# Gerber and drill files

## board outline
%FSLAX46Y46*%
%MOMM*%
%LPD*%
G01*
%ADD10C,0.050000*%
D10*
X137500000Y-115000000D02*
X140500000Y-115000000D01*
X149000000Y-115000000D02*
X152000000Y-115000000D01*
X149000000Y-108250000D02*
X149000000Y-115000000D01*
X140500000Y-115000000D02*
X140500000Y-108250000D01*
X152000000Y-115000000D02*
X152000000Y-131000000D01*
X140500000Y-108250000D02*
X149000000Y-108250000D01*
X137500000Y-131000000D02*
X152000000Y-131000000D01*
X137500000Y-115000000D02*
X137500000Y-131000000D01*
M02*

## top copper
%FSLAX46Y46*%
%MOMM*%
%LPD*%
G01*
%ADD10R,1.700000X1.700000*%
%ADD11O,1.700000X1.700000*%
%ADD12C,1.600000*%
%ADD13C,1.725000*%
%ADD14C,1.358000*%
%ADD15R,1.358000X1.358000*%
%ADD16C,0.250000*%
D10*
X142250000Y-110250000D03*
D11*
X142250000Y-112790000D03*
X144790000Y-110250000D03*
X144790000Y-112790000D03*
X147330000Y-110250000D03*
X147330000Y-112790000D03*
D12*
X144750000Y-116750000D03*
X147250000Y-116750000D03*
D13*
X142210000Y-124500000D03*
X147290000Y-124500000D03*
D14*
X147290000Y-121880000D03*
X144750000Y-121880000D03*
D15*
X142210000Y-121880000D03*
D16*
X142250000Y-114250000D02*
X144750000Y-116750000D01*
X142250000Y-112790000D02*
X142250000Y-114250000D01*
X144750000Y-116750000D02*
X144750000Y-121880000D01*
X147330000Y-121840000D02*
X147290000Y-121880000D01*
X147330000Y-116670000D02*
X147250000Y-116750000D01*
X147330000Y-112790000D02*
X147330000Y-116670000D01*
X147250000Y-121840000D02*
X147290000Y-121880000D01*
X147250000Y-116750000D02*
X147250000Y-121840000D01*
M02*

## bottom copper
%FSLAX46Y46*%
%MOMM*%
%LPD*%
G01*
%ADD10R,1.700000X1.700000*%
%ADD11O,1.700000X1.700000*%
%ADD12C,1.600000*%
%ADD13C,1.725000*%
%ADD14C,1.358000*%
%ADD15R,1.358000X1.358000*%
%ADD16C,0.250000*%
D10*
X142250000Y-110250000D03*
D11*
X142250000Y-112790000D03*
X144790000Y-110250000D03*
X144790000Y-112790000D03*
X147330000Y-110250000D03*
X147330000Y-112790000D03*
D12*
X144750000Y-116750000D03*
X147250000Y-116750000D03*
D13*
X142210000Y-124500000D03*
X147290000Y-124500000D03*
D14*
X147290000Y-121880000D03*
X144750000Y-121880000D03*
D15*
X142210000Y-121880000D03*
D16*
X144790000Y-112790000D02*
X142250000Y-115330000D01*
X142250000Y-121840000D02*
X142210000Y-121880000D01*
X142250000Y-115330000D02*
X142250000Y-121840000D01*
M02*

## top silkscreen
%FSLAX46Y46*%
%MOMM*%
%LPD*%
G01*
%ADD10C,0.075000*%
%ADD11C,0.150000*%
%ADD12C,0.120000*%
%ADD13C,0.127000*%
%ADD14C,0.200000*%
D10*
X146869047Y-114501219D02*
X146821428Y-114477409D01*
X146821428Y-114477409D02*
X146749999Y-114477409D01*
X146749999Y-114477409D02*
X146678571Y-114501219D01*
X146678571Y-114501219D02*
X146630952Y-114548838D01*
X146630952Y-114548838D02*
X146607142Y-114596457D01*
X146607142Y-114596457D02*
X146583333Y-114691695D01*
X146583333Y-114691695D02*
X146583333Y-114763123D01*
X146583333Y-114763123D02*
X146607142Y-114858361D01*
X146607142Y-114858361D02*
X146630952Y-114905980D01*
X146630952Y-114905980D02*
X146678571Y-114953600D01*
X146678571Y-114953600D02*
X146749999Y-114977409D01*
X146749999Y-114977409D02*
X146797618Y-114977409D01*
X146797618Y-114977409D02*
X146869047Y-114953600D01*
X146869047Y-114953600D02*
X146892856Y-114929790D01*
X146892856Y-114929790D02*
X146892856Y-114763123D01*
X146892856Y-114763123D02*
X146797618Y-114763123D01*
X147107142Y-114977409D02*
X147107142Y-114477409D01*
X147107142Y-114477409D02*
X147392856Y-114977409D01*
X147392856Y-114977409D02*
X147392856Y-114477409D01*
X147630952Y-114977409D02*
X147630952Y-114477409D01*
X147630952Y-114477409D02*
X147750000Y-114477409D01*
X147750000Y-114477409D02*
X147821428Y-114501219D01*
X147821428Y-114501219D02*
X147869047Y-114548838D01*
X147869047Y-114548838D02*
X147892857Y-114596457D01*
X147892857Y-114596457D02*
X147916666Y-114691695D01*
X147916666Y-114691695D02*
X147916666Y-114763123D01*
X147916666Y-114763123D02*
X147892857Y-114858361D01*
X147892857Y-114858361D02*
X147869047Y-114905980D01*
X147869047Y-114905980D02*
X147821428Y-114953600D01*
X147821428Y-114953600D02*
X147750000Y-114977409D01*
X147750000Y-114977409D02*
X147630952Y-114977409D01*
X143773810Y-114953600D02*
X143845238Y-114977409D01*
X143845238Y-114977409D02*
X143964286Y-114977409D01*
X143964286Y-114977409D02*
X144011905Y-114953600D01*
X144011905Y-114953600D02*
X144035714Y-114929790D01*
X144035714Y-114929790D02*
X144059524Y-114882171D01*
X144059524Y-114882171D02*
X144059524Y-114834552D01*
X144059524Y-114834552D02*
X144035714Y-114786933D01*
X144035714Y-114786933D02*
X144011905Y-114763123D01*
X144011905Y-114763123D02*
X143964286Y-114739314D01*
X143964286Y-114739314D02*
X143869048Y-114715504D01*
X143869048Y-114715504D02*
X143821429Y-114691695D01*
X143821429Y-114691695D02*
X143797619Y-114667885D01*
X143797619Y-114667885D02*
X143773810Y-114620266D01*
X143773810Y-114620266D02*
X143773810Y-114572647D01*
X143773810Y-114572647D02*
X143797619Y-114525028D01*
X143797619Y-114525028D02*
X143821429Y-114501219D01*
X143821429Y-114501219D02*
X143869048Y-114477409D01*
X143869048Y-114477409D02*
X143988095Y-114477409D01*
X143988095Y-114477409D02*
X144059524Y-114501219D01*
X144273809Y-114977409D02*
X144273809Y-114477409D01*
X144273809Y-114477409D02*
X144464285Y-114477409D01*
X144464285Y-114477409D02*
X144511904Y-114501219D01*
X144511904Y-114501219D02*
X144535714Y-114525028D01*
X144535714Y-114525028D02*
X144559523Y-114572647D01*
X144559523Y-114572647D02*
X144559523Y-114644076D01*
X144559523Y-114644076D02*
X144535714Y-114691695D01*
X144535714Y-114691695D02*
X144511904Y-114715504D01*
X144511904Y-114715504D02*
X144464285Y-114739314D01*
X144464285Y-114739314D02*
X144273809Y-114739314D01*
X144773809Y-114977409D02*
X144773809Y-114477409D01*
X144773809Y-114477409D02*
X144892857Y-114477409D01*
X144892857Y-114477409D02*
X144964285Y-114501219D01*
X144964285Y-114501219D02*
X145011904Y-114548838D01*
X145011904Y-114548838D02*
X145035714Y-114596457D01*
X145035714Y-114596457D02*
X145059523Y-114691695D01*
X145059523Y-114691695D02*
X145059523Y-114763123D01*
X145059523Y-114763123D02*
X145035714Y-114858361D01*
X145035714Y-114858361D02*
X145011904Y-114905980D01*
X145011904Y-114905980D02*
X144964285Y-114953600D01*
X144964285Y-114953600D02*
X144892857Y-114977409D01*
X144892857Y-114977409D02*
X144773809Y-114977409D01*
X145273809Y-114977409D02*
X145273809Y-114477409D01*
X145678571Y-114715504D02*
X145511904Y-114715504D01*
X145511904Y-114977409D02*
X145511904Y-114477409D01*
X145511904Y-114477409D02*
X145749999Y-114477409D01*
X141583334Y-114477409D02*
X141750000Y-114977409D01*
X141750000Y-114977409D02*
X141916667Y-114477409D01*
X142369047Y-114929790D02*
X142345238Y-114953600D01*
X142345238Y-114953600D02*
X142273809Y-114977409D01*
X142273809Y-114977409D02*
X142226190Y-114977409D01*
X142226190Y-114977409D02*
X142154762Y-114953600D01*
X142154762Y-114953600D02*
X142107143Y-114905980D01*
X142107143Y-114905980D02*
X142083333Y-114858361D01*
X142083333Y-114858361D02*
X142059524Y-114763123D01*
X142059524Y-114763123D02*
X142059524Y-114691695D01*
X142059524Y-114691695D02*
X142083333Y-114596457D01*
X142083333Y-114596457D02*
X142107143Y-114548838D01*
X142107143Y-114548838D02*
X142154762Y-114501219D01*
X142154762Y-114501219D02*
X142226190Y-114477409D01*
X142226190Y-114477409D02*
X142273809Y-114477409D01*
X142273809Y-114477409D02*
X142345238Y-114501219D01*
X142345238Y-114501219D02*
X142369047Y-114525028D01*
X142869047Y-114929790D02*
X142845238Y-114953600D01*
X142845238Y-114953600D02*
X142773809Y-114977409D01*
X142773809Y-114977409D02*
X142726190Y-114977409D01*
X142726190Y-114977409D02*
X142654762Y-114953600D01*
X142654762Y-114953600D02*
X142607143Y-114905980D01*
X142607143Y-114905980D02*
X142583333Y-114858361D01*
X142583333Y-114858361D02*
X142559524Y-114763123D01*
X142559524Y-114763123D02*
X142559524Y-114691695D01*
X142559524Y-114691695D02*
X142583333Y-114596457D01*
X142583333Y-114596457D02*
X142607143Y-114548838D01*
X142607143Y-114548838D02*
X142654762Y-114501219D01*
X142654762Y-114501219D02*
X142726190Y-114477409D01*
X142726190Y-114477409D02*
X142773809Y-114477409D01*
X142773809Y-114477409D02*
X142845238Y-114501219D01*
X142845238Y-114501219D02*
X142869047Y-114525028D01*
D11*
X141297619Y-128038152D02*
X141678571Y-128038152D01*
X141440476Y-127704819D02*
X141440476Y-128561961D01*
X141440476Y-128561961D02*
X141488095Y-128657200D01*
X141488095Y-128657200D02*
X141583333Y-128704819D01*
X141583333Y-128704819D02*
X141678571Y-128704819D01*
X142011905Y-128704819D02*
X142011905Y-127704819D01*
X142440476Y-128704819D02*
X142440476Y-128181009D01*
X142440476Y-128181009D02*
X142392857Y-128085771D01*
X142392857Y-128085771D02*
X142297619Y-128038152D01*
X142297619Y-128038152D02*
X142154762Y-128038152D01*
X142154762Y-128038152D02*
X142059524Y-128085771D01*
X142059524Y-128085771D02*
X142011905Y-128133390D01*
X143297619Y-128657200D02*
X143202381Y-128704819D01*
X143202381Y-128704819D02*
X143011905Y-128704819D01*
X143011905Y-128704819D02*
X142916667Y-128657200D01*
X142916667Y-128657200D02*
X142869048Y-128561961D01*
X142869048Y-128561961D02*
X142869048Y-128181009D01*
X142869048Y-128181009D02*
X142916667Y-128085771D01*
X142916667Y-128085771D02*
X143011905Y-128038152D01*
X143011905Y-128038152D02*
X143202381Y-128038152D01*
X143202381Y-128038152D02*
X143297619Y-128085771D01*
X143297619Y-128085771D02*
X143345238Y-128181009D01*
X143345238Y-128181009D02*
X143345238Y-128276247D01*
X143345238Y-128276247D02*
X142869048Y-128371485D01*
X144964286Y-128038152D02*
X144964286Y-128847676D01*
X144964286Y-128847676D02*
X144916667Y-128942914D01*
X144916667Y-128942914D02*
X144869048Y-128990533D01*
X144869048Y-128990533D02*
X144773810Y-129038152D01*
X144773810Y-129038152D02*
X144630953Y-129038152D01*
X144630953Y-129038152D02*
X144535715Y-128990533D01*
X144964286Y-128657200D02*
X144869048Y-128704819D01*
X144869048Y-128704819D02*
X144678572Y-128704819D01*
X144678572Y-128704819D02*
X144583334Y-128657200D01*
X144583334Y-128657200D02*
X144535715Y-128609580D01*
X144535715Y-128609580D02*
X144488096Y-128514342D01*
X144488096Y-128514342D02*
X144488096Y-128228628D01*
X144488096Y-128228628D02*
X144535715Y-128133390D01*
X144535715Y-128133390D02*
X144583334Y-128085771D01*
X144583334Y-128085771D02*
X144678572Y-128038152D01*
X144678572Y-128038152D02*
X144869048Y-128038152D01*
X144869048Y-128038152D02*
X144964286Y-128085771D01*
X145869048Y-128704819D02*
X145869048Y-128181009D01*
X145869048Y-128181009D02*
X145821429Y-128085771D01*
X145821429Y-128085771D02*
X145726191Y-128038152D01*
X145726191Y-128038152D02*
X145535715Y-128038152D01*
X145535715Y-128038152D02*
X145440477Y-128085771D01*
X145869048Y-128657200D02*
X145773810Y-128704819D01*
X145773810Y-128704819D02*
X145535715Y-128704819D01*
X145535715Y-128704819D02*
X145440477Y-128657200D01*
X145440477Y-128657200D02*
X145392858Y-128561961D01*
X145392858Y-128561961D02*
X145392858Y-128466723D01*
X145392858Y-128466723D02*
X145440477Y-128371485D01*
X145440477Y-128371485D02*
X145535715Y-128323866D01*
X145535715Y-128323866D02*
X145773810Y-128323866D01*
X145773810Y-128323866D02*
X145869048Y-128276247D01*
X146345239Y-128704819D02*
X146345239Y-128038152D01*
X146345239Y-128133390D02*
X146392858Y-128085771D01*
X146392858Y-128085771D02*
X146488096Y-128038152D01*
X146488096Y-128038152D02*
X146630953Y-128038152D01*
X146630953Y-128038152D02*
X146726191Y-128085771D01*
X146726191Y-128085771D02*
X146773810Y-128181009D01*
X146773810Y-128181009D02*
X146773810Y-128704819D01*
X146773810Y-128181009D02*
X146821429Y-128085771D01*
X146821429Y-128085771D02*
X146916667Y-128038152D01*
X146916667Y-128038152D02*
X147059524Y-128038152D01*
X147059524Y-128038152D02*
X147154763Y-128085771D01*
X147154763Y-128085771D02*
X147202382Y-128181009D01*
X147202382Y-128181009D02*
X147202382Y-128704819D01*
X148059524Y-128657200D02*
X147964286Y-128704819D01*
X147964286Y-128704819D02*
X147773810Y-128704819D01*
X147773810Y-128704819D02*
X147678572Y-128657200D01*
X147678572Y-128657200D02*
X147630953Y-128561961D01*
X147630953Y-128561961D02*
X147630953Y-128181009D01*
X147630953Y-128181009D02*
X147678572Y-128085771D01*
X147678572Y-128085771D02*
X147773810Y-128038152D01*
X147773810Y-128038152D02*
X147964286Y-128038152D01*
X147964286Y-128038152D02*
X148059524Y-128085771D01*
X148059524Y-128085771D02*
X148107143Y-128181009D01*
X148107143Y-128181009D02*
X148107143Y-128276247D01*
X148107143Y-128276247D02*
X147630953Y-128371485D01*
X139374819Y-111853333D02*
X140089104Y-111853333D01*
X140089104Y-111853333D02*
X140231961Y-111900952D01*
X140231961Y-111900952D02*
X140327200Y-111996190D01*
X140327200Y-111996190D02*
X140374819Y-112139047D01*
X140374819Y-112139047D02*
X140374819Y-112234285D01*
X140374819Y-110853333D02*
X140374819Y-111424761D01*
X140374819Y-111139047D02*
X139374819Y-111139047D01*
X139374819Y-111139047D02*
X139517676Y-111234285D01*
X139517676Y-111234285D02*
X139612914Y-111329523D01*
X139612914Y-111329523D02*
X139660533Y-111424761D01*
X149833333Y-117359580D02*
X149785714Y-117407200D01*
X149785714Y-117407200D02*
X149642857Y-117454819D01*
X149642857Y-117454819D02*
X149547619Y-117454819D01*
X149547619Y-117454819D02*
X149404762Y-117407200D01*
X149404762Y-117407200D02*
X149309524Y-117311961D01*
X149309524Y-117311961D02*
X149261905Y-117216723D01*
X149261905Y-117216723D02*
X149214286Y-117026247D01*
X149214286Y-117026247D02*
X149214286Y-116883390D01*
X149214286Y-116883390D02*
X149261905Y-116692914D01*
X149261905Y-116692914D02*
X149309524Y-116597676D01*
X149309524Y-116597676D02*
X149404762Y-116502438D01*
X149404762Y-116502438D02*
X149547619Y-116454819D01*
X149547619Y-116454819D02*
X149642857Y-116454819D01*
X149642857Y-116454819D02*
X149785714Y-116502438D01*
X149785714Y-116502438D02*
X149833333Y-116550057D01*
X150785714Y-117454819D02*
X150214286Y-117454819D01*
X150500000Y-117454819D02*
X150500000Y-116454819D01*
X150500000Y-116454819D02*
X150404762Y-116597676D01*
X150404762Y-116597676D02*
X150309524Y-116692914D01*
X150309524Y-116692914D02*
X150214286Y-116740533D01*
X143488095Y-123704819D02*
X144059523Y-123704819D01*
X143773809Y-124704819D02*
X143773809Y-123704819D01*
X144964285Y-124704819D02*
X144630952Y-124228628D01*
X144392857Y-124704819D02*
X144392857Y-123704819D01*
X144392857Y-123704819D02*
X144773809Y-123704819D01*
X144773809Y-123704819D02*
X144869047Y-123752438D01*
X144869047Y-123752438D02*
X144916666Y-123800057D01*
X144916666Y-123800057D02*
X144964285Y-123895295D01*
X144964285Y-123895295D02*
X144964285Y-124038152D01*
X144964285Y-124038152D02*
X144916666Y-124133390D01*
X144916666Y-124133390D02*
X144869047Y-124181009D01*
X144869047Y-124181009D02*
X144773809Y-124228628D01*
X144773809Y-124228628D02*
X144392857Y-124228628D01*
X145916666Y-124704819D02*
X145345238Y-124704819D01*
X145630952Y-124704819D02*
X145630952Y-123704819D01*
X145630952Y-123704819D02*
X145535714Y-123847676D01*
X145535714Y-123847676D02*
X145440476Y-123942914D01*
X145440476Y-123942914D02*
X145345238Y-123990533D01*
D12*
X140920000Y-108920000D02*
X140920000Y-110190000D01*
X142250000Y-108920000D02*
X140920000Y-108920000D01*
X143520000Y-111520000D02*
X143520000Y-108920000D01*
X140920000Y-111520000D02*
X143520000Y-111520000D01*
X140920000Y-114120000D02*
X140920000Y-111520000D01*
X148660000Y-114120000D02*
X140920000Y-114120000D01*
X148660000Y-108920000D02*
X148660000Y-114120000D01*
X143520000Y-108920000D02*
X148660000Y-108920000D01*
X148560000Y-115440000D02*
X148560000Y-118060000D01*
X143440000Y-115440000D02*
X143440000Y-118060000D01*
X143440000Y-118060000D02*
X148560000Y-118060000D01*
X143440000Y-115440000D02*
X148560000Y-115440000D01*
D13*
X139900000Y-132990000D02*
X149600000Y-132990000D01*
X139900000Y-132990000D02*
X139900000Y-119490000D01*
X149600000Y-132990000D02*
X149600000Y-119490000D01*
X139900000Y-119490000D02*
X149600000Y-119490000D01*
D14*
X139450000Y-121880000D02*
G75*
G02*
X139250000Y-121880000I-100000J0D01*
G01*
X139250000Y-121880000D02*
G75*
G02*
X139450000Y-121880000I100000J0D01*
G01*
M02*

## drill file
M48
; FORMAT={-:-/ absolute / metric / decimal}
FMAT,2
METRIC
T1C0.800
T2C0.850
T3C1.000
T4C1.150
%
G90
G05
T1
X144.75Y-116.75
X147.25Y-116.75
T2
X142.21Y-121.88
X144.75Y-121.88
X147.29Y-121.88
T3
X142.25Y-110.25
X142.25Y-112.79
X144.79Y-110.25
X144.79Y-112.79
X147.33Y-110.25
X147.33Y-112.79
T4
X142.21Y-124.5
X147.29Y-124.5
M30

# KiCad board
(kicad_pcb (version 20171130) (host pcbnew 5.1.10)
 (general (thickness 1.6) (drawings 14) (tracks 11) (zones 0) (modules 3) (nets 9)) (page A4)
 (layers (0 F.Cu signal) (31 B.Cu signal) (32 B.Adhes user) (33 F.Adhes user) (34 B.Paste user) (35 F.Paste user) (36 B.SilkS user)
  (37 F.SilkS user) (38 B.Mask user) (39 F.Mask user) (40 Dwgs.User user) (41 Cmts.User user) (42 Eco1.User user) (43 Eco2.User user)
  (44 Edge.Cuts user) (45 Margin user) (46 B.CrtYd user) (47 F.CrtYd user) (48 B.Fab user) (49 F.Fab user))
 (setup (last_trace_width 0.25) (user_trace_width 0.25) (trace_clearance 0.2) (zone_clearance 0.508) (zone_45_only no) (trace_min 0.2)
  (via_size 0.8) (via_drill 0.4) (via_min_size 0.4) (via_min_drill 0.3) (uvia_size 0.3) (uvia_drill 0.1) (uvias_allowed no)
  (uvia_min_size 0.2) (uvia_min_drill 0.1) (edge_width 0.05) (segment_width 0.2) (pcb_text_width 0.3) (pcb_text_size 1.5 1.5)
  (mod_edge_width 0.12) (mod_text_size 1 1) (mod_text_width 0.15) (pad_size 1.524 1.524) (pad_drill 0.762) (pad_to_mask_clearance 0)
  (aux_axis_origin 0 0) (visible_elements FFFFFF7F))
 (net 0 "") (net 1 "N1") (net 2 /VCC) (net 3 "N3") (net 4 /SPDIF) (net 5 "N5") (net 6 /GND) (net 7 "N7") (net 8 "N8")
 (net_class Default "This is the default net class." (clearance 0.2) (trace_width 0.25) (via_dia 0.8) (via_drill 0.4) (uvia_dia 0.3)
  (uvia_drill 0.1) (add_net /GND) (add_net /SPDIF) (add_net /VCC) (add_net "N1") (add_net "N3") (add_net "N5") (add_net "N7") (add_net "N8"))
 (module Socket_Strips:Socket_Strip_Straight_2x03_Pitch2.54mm (layer F.Cu) (at 142.25 110.25 90)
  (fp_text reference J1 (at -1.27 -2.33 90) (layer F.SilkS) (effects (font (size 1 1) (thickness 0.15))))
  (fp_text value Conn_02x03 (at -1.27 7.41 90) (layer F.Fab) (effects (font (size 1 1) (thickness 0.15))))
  (fp_line (start 1.33 -1.33) (end 0.06 -1.33) (layer F.SilkS) (width 0.12))
  (fp_line (start 1.33 0) (end 1.33 -1.33) (layer F.SilkS) (width 0.12))
  (fp_line (start -1.27 1.27) (end 1.33 1.27) (layer F.SilkS) (width 0.12))
  (fp_line (start -1.27 -1.33) (end -1.27 1.27) (layer F.SilkS) (width 0.12))
  (fp_line (start -3.87 -1.33) (end -1.27 -1.33) (layer F.SilkS) (width 0.12))
  (fp_line (start -3.87 6.41) (end -3.87 -1.33) (layer F.SilkS) (width 0.12))
  (fp_line (start 1.33 6.41) (end -3.87 6.41) (layer F.SilkS) (width 0.12))
  (fp_line (start 1.33 1.27) (end 1.33 6.41) (layer F.SilkS) (width 0.12))
  (pad 1 thru_hole rect (at 0 0 90) (size 1.7 1.7) (drill 1) (layers *.Cu *.Mask) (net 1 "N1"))
  (pad 2 thru_hole oval (at -2.54 0 90) (size 1.7 1.7) (drill 1) (layers *.Cu *.Mask) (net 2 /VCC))
  (pad 3 thru_hole oval (at 0 2.54 90) (size 1.7 1.7) (drill 1) (layers *.Cu *.Mask) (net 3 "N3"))
  (pad 4 thru_hole oval (at -2.54 2.54 90) (size 1.7 1.7) (drill 1) (layers *.Cu *.Mask) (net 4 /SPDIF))
  (pad 5 thru_hole oval (at 0 5.08 90) (size 1.7 1.7) (drill 1) (layers *.Cu *.Mask) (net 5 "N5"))
  (pad 6 thru_hole oval (at -2.54 5.08 90) (size 1.7 1.7) (drill 1) (layers *.Cu *.Mask) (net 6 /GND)))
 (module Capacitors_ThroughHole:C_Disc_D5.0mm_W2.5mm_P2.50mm (layer F.Cu) (at 144.75 116.75)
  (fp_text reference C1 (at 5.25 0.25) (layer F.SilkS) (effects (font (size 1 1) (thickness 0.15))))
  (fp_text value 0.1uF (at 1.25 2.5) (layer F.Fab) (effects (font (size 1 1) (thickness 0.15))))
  (fp_line (start 3.81 -1.31) (end 3.81 1.31) (layer F.SilkS) (width 0.12))
  (fp_line (start -1.31 -1.31) (end -1.31 1.31) (layer F.SilkS) (width 0.12))
  (fp_line (start -1.31 1.31) (end 3.81 1.31) (layer F.SilkS) (width 0.12))
  (fp_line (start -1.31 -1.31) (end 3.81 -1.31) (layer F.SilkS) (width 0.12))
  (pad 1 thru_hole circle (at 0 0) (size 1.6 1.6) (drill 0.8) (layers *.Cu *.Mask) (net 2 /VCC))
  (pad 2 thru_hole circle (at 2.5 0) (size 1.6 1.6) (drill 0.8) (layers *.Cu *.Mask) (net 6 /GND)))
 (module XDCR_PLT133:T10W (layer F.Cu) (at 144.75 124.5)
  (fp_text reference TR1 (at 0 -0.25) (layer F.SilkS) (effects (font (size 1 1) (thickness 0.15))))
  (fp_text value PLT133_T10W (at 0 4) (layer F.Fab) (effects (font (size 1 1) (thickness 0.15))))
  (fp_line (start -4.85 8.49) (end 4.85 8.49) (layer F.SilkS) (width 0.127))
  (fp_line (start -4.85 8.49) (end -4.85 -5.01) (layer F.SilkS) (width 0.127))
  (fp_line (start 4.85 8.49) (end 4.85 -5.01) (layer F.SilkS) (width 0.127))
  (fp_line (start -4.85 -5.01) (end 4.85 -5.01) (layer F.SilkS) (width 0.127))
  (fp_circle (center -5.4 -2.62) (end -5.3 -2.62) (layer F.SilkS) (width 0.2))
  (pad 4 thru_hole circle (at -2.54 0) (size 1.725 1.725) (drill 1.15) (layers *.Cu *.Mask) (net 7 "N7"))
  (pad 5 thru_hole circle (at 2.54 0) (size 1.725 1.725) (drill 1.15) (layers *.Cu *.Mask) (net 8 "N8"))
  (pad 3 thru_hole circle (at 2.54 -2.62) (size 1.358 1.358) (drill 0.85) (layers *.Cu *.Mask) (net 6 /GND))
  (pad 2 thru_hole circle (at 0 -2.62) (size 1.358 1.358) (drill 0.85) (layers *.Cu *.Mask) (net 2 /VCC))
  (pad 1 thru_hole rect (at -2.54 -2.62) (size 1.358 1.358) (drill 0.85) (layers *.Cu *.Mask) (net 4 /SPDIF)))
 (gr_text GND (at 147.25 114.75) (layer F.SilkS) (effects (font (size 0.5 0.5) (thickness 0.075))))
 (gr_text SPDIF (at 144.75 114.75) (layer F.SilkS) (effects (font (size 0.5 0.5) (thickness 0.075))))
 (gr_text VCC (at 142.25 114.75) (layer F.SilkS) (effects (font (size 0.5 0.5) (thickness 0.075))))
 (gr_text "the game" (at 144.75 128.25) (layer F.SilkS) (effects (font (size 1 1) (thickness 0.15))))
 (gr_line (start 137.5 115) (end 140.5 115) (layer Edge.Cuts) (width 0.05))
 (gr_line (start 149 115) (end 152 115) (layer Edge.Cuts) (width 0.05))
 (gr_line (start 149 108.25) (end 149 115) (layer Edge.Cuts) (width 0.05))
 (gr_line (start 140.5 115) (end 140.5 108.25) (layer Edge.Cuts) (width 0.05))
 (gr_line (start 152 115) (end 152 131) (layer Edge.Cuts) (width 0.05))
 (gr_line (start 140.5 108.25) (end 149 108.25) (layer Edge.Cuts) (width 0.05))
 (gr_line (start 137.5 131) (end 152 131) (layer Edge.Cuts) (width 0.05))
 (gr_line (start 137.5 115) (end 137.5 131) (layer Edge.Cuts) (width 0.05))
 (segment (start 144.79 112.79) (end 142.25 115.33) (width 0.25) (layer B.Cu) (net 4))
 (segment (start 142.25 121.84) (end 142.21 121.88) (width 0.25) (layer B.Cu) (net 4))
 (segment (start 142.25 115.33) (end 142.25 121.84) (width 0.25) (layer B.Cu) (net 4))
 (segment (start 142.25 114.25) (end 144.75 116.75) (width 0.25) (layer F.Cu) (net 2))
 (segment (start 142.25 112.79) (end 142.25 114.25) (width 0.25) (layer F.Cu) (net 2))
 (segment (start 144.75 116.75) (end 144.75 121.88) (width 0.25) (layer F.Cu) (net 2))
 (segment (start 147.33 121.84) (end 147.29 121.88) (width 0.25) (layer F.Cu) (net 6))
 (segment (start 147.33 116.67) (end 147.25 116.75) (width 0.25) (layer F.Cu) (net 6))
 (segment (start 147.33 112.79) (end 147.33 116.67) (width 0.25) (layer F.Cu) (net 6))
 (segment (start 147.25 121.84) (end 147.29 121.88) (width 0.25) (layer F.Cu) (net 6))
 (segment (start 147.25 116.75) (end 147.25 121.84) (width 0.25) (layer F.Cu) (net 6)))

